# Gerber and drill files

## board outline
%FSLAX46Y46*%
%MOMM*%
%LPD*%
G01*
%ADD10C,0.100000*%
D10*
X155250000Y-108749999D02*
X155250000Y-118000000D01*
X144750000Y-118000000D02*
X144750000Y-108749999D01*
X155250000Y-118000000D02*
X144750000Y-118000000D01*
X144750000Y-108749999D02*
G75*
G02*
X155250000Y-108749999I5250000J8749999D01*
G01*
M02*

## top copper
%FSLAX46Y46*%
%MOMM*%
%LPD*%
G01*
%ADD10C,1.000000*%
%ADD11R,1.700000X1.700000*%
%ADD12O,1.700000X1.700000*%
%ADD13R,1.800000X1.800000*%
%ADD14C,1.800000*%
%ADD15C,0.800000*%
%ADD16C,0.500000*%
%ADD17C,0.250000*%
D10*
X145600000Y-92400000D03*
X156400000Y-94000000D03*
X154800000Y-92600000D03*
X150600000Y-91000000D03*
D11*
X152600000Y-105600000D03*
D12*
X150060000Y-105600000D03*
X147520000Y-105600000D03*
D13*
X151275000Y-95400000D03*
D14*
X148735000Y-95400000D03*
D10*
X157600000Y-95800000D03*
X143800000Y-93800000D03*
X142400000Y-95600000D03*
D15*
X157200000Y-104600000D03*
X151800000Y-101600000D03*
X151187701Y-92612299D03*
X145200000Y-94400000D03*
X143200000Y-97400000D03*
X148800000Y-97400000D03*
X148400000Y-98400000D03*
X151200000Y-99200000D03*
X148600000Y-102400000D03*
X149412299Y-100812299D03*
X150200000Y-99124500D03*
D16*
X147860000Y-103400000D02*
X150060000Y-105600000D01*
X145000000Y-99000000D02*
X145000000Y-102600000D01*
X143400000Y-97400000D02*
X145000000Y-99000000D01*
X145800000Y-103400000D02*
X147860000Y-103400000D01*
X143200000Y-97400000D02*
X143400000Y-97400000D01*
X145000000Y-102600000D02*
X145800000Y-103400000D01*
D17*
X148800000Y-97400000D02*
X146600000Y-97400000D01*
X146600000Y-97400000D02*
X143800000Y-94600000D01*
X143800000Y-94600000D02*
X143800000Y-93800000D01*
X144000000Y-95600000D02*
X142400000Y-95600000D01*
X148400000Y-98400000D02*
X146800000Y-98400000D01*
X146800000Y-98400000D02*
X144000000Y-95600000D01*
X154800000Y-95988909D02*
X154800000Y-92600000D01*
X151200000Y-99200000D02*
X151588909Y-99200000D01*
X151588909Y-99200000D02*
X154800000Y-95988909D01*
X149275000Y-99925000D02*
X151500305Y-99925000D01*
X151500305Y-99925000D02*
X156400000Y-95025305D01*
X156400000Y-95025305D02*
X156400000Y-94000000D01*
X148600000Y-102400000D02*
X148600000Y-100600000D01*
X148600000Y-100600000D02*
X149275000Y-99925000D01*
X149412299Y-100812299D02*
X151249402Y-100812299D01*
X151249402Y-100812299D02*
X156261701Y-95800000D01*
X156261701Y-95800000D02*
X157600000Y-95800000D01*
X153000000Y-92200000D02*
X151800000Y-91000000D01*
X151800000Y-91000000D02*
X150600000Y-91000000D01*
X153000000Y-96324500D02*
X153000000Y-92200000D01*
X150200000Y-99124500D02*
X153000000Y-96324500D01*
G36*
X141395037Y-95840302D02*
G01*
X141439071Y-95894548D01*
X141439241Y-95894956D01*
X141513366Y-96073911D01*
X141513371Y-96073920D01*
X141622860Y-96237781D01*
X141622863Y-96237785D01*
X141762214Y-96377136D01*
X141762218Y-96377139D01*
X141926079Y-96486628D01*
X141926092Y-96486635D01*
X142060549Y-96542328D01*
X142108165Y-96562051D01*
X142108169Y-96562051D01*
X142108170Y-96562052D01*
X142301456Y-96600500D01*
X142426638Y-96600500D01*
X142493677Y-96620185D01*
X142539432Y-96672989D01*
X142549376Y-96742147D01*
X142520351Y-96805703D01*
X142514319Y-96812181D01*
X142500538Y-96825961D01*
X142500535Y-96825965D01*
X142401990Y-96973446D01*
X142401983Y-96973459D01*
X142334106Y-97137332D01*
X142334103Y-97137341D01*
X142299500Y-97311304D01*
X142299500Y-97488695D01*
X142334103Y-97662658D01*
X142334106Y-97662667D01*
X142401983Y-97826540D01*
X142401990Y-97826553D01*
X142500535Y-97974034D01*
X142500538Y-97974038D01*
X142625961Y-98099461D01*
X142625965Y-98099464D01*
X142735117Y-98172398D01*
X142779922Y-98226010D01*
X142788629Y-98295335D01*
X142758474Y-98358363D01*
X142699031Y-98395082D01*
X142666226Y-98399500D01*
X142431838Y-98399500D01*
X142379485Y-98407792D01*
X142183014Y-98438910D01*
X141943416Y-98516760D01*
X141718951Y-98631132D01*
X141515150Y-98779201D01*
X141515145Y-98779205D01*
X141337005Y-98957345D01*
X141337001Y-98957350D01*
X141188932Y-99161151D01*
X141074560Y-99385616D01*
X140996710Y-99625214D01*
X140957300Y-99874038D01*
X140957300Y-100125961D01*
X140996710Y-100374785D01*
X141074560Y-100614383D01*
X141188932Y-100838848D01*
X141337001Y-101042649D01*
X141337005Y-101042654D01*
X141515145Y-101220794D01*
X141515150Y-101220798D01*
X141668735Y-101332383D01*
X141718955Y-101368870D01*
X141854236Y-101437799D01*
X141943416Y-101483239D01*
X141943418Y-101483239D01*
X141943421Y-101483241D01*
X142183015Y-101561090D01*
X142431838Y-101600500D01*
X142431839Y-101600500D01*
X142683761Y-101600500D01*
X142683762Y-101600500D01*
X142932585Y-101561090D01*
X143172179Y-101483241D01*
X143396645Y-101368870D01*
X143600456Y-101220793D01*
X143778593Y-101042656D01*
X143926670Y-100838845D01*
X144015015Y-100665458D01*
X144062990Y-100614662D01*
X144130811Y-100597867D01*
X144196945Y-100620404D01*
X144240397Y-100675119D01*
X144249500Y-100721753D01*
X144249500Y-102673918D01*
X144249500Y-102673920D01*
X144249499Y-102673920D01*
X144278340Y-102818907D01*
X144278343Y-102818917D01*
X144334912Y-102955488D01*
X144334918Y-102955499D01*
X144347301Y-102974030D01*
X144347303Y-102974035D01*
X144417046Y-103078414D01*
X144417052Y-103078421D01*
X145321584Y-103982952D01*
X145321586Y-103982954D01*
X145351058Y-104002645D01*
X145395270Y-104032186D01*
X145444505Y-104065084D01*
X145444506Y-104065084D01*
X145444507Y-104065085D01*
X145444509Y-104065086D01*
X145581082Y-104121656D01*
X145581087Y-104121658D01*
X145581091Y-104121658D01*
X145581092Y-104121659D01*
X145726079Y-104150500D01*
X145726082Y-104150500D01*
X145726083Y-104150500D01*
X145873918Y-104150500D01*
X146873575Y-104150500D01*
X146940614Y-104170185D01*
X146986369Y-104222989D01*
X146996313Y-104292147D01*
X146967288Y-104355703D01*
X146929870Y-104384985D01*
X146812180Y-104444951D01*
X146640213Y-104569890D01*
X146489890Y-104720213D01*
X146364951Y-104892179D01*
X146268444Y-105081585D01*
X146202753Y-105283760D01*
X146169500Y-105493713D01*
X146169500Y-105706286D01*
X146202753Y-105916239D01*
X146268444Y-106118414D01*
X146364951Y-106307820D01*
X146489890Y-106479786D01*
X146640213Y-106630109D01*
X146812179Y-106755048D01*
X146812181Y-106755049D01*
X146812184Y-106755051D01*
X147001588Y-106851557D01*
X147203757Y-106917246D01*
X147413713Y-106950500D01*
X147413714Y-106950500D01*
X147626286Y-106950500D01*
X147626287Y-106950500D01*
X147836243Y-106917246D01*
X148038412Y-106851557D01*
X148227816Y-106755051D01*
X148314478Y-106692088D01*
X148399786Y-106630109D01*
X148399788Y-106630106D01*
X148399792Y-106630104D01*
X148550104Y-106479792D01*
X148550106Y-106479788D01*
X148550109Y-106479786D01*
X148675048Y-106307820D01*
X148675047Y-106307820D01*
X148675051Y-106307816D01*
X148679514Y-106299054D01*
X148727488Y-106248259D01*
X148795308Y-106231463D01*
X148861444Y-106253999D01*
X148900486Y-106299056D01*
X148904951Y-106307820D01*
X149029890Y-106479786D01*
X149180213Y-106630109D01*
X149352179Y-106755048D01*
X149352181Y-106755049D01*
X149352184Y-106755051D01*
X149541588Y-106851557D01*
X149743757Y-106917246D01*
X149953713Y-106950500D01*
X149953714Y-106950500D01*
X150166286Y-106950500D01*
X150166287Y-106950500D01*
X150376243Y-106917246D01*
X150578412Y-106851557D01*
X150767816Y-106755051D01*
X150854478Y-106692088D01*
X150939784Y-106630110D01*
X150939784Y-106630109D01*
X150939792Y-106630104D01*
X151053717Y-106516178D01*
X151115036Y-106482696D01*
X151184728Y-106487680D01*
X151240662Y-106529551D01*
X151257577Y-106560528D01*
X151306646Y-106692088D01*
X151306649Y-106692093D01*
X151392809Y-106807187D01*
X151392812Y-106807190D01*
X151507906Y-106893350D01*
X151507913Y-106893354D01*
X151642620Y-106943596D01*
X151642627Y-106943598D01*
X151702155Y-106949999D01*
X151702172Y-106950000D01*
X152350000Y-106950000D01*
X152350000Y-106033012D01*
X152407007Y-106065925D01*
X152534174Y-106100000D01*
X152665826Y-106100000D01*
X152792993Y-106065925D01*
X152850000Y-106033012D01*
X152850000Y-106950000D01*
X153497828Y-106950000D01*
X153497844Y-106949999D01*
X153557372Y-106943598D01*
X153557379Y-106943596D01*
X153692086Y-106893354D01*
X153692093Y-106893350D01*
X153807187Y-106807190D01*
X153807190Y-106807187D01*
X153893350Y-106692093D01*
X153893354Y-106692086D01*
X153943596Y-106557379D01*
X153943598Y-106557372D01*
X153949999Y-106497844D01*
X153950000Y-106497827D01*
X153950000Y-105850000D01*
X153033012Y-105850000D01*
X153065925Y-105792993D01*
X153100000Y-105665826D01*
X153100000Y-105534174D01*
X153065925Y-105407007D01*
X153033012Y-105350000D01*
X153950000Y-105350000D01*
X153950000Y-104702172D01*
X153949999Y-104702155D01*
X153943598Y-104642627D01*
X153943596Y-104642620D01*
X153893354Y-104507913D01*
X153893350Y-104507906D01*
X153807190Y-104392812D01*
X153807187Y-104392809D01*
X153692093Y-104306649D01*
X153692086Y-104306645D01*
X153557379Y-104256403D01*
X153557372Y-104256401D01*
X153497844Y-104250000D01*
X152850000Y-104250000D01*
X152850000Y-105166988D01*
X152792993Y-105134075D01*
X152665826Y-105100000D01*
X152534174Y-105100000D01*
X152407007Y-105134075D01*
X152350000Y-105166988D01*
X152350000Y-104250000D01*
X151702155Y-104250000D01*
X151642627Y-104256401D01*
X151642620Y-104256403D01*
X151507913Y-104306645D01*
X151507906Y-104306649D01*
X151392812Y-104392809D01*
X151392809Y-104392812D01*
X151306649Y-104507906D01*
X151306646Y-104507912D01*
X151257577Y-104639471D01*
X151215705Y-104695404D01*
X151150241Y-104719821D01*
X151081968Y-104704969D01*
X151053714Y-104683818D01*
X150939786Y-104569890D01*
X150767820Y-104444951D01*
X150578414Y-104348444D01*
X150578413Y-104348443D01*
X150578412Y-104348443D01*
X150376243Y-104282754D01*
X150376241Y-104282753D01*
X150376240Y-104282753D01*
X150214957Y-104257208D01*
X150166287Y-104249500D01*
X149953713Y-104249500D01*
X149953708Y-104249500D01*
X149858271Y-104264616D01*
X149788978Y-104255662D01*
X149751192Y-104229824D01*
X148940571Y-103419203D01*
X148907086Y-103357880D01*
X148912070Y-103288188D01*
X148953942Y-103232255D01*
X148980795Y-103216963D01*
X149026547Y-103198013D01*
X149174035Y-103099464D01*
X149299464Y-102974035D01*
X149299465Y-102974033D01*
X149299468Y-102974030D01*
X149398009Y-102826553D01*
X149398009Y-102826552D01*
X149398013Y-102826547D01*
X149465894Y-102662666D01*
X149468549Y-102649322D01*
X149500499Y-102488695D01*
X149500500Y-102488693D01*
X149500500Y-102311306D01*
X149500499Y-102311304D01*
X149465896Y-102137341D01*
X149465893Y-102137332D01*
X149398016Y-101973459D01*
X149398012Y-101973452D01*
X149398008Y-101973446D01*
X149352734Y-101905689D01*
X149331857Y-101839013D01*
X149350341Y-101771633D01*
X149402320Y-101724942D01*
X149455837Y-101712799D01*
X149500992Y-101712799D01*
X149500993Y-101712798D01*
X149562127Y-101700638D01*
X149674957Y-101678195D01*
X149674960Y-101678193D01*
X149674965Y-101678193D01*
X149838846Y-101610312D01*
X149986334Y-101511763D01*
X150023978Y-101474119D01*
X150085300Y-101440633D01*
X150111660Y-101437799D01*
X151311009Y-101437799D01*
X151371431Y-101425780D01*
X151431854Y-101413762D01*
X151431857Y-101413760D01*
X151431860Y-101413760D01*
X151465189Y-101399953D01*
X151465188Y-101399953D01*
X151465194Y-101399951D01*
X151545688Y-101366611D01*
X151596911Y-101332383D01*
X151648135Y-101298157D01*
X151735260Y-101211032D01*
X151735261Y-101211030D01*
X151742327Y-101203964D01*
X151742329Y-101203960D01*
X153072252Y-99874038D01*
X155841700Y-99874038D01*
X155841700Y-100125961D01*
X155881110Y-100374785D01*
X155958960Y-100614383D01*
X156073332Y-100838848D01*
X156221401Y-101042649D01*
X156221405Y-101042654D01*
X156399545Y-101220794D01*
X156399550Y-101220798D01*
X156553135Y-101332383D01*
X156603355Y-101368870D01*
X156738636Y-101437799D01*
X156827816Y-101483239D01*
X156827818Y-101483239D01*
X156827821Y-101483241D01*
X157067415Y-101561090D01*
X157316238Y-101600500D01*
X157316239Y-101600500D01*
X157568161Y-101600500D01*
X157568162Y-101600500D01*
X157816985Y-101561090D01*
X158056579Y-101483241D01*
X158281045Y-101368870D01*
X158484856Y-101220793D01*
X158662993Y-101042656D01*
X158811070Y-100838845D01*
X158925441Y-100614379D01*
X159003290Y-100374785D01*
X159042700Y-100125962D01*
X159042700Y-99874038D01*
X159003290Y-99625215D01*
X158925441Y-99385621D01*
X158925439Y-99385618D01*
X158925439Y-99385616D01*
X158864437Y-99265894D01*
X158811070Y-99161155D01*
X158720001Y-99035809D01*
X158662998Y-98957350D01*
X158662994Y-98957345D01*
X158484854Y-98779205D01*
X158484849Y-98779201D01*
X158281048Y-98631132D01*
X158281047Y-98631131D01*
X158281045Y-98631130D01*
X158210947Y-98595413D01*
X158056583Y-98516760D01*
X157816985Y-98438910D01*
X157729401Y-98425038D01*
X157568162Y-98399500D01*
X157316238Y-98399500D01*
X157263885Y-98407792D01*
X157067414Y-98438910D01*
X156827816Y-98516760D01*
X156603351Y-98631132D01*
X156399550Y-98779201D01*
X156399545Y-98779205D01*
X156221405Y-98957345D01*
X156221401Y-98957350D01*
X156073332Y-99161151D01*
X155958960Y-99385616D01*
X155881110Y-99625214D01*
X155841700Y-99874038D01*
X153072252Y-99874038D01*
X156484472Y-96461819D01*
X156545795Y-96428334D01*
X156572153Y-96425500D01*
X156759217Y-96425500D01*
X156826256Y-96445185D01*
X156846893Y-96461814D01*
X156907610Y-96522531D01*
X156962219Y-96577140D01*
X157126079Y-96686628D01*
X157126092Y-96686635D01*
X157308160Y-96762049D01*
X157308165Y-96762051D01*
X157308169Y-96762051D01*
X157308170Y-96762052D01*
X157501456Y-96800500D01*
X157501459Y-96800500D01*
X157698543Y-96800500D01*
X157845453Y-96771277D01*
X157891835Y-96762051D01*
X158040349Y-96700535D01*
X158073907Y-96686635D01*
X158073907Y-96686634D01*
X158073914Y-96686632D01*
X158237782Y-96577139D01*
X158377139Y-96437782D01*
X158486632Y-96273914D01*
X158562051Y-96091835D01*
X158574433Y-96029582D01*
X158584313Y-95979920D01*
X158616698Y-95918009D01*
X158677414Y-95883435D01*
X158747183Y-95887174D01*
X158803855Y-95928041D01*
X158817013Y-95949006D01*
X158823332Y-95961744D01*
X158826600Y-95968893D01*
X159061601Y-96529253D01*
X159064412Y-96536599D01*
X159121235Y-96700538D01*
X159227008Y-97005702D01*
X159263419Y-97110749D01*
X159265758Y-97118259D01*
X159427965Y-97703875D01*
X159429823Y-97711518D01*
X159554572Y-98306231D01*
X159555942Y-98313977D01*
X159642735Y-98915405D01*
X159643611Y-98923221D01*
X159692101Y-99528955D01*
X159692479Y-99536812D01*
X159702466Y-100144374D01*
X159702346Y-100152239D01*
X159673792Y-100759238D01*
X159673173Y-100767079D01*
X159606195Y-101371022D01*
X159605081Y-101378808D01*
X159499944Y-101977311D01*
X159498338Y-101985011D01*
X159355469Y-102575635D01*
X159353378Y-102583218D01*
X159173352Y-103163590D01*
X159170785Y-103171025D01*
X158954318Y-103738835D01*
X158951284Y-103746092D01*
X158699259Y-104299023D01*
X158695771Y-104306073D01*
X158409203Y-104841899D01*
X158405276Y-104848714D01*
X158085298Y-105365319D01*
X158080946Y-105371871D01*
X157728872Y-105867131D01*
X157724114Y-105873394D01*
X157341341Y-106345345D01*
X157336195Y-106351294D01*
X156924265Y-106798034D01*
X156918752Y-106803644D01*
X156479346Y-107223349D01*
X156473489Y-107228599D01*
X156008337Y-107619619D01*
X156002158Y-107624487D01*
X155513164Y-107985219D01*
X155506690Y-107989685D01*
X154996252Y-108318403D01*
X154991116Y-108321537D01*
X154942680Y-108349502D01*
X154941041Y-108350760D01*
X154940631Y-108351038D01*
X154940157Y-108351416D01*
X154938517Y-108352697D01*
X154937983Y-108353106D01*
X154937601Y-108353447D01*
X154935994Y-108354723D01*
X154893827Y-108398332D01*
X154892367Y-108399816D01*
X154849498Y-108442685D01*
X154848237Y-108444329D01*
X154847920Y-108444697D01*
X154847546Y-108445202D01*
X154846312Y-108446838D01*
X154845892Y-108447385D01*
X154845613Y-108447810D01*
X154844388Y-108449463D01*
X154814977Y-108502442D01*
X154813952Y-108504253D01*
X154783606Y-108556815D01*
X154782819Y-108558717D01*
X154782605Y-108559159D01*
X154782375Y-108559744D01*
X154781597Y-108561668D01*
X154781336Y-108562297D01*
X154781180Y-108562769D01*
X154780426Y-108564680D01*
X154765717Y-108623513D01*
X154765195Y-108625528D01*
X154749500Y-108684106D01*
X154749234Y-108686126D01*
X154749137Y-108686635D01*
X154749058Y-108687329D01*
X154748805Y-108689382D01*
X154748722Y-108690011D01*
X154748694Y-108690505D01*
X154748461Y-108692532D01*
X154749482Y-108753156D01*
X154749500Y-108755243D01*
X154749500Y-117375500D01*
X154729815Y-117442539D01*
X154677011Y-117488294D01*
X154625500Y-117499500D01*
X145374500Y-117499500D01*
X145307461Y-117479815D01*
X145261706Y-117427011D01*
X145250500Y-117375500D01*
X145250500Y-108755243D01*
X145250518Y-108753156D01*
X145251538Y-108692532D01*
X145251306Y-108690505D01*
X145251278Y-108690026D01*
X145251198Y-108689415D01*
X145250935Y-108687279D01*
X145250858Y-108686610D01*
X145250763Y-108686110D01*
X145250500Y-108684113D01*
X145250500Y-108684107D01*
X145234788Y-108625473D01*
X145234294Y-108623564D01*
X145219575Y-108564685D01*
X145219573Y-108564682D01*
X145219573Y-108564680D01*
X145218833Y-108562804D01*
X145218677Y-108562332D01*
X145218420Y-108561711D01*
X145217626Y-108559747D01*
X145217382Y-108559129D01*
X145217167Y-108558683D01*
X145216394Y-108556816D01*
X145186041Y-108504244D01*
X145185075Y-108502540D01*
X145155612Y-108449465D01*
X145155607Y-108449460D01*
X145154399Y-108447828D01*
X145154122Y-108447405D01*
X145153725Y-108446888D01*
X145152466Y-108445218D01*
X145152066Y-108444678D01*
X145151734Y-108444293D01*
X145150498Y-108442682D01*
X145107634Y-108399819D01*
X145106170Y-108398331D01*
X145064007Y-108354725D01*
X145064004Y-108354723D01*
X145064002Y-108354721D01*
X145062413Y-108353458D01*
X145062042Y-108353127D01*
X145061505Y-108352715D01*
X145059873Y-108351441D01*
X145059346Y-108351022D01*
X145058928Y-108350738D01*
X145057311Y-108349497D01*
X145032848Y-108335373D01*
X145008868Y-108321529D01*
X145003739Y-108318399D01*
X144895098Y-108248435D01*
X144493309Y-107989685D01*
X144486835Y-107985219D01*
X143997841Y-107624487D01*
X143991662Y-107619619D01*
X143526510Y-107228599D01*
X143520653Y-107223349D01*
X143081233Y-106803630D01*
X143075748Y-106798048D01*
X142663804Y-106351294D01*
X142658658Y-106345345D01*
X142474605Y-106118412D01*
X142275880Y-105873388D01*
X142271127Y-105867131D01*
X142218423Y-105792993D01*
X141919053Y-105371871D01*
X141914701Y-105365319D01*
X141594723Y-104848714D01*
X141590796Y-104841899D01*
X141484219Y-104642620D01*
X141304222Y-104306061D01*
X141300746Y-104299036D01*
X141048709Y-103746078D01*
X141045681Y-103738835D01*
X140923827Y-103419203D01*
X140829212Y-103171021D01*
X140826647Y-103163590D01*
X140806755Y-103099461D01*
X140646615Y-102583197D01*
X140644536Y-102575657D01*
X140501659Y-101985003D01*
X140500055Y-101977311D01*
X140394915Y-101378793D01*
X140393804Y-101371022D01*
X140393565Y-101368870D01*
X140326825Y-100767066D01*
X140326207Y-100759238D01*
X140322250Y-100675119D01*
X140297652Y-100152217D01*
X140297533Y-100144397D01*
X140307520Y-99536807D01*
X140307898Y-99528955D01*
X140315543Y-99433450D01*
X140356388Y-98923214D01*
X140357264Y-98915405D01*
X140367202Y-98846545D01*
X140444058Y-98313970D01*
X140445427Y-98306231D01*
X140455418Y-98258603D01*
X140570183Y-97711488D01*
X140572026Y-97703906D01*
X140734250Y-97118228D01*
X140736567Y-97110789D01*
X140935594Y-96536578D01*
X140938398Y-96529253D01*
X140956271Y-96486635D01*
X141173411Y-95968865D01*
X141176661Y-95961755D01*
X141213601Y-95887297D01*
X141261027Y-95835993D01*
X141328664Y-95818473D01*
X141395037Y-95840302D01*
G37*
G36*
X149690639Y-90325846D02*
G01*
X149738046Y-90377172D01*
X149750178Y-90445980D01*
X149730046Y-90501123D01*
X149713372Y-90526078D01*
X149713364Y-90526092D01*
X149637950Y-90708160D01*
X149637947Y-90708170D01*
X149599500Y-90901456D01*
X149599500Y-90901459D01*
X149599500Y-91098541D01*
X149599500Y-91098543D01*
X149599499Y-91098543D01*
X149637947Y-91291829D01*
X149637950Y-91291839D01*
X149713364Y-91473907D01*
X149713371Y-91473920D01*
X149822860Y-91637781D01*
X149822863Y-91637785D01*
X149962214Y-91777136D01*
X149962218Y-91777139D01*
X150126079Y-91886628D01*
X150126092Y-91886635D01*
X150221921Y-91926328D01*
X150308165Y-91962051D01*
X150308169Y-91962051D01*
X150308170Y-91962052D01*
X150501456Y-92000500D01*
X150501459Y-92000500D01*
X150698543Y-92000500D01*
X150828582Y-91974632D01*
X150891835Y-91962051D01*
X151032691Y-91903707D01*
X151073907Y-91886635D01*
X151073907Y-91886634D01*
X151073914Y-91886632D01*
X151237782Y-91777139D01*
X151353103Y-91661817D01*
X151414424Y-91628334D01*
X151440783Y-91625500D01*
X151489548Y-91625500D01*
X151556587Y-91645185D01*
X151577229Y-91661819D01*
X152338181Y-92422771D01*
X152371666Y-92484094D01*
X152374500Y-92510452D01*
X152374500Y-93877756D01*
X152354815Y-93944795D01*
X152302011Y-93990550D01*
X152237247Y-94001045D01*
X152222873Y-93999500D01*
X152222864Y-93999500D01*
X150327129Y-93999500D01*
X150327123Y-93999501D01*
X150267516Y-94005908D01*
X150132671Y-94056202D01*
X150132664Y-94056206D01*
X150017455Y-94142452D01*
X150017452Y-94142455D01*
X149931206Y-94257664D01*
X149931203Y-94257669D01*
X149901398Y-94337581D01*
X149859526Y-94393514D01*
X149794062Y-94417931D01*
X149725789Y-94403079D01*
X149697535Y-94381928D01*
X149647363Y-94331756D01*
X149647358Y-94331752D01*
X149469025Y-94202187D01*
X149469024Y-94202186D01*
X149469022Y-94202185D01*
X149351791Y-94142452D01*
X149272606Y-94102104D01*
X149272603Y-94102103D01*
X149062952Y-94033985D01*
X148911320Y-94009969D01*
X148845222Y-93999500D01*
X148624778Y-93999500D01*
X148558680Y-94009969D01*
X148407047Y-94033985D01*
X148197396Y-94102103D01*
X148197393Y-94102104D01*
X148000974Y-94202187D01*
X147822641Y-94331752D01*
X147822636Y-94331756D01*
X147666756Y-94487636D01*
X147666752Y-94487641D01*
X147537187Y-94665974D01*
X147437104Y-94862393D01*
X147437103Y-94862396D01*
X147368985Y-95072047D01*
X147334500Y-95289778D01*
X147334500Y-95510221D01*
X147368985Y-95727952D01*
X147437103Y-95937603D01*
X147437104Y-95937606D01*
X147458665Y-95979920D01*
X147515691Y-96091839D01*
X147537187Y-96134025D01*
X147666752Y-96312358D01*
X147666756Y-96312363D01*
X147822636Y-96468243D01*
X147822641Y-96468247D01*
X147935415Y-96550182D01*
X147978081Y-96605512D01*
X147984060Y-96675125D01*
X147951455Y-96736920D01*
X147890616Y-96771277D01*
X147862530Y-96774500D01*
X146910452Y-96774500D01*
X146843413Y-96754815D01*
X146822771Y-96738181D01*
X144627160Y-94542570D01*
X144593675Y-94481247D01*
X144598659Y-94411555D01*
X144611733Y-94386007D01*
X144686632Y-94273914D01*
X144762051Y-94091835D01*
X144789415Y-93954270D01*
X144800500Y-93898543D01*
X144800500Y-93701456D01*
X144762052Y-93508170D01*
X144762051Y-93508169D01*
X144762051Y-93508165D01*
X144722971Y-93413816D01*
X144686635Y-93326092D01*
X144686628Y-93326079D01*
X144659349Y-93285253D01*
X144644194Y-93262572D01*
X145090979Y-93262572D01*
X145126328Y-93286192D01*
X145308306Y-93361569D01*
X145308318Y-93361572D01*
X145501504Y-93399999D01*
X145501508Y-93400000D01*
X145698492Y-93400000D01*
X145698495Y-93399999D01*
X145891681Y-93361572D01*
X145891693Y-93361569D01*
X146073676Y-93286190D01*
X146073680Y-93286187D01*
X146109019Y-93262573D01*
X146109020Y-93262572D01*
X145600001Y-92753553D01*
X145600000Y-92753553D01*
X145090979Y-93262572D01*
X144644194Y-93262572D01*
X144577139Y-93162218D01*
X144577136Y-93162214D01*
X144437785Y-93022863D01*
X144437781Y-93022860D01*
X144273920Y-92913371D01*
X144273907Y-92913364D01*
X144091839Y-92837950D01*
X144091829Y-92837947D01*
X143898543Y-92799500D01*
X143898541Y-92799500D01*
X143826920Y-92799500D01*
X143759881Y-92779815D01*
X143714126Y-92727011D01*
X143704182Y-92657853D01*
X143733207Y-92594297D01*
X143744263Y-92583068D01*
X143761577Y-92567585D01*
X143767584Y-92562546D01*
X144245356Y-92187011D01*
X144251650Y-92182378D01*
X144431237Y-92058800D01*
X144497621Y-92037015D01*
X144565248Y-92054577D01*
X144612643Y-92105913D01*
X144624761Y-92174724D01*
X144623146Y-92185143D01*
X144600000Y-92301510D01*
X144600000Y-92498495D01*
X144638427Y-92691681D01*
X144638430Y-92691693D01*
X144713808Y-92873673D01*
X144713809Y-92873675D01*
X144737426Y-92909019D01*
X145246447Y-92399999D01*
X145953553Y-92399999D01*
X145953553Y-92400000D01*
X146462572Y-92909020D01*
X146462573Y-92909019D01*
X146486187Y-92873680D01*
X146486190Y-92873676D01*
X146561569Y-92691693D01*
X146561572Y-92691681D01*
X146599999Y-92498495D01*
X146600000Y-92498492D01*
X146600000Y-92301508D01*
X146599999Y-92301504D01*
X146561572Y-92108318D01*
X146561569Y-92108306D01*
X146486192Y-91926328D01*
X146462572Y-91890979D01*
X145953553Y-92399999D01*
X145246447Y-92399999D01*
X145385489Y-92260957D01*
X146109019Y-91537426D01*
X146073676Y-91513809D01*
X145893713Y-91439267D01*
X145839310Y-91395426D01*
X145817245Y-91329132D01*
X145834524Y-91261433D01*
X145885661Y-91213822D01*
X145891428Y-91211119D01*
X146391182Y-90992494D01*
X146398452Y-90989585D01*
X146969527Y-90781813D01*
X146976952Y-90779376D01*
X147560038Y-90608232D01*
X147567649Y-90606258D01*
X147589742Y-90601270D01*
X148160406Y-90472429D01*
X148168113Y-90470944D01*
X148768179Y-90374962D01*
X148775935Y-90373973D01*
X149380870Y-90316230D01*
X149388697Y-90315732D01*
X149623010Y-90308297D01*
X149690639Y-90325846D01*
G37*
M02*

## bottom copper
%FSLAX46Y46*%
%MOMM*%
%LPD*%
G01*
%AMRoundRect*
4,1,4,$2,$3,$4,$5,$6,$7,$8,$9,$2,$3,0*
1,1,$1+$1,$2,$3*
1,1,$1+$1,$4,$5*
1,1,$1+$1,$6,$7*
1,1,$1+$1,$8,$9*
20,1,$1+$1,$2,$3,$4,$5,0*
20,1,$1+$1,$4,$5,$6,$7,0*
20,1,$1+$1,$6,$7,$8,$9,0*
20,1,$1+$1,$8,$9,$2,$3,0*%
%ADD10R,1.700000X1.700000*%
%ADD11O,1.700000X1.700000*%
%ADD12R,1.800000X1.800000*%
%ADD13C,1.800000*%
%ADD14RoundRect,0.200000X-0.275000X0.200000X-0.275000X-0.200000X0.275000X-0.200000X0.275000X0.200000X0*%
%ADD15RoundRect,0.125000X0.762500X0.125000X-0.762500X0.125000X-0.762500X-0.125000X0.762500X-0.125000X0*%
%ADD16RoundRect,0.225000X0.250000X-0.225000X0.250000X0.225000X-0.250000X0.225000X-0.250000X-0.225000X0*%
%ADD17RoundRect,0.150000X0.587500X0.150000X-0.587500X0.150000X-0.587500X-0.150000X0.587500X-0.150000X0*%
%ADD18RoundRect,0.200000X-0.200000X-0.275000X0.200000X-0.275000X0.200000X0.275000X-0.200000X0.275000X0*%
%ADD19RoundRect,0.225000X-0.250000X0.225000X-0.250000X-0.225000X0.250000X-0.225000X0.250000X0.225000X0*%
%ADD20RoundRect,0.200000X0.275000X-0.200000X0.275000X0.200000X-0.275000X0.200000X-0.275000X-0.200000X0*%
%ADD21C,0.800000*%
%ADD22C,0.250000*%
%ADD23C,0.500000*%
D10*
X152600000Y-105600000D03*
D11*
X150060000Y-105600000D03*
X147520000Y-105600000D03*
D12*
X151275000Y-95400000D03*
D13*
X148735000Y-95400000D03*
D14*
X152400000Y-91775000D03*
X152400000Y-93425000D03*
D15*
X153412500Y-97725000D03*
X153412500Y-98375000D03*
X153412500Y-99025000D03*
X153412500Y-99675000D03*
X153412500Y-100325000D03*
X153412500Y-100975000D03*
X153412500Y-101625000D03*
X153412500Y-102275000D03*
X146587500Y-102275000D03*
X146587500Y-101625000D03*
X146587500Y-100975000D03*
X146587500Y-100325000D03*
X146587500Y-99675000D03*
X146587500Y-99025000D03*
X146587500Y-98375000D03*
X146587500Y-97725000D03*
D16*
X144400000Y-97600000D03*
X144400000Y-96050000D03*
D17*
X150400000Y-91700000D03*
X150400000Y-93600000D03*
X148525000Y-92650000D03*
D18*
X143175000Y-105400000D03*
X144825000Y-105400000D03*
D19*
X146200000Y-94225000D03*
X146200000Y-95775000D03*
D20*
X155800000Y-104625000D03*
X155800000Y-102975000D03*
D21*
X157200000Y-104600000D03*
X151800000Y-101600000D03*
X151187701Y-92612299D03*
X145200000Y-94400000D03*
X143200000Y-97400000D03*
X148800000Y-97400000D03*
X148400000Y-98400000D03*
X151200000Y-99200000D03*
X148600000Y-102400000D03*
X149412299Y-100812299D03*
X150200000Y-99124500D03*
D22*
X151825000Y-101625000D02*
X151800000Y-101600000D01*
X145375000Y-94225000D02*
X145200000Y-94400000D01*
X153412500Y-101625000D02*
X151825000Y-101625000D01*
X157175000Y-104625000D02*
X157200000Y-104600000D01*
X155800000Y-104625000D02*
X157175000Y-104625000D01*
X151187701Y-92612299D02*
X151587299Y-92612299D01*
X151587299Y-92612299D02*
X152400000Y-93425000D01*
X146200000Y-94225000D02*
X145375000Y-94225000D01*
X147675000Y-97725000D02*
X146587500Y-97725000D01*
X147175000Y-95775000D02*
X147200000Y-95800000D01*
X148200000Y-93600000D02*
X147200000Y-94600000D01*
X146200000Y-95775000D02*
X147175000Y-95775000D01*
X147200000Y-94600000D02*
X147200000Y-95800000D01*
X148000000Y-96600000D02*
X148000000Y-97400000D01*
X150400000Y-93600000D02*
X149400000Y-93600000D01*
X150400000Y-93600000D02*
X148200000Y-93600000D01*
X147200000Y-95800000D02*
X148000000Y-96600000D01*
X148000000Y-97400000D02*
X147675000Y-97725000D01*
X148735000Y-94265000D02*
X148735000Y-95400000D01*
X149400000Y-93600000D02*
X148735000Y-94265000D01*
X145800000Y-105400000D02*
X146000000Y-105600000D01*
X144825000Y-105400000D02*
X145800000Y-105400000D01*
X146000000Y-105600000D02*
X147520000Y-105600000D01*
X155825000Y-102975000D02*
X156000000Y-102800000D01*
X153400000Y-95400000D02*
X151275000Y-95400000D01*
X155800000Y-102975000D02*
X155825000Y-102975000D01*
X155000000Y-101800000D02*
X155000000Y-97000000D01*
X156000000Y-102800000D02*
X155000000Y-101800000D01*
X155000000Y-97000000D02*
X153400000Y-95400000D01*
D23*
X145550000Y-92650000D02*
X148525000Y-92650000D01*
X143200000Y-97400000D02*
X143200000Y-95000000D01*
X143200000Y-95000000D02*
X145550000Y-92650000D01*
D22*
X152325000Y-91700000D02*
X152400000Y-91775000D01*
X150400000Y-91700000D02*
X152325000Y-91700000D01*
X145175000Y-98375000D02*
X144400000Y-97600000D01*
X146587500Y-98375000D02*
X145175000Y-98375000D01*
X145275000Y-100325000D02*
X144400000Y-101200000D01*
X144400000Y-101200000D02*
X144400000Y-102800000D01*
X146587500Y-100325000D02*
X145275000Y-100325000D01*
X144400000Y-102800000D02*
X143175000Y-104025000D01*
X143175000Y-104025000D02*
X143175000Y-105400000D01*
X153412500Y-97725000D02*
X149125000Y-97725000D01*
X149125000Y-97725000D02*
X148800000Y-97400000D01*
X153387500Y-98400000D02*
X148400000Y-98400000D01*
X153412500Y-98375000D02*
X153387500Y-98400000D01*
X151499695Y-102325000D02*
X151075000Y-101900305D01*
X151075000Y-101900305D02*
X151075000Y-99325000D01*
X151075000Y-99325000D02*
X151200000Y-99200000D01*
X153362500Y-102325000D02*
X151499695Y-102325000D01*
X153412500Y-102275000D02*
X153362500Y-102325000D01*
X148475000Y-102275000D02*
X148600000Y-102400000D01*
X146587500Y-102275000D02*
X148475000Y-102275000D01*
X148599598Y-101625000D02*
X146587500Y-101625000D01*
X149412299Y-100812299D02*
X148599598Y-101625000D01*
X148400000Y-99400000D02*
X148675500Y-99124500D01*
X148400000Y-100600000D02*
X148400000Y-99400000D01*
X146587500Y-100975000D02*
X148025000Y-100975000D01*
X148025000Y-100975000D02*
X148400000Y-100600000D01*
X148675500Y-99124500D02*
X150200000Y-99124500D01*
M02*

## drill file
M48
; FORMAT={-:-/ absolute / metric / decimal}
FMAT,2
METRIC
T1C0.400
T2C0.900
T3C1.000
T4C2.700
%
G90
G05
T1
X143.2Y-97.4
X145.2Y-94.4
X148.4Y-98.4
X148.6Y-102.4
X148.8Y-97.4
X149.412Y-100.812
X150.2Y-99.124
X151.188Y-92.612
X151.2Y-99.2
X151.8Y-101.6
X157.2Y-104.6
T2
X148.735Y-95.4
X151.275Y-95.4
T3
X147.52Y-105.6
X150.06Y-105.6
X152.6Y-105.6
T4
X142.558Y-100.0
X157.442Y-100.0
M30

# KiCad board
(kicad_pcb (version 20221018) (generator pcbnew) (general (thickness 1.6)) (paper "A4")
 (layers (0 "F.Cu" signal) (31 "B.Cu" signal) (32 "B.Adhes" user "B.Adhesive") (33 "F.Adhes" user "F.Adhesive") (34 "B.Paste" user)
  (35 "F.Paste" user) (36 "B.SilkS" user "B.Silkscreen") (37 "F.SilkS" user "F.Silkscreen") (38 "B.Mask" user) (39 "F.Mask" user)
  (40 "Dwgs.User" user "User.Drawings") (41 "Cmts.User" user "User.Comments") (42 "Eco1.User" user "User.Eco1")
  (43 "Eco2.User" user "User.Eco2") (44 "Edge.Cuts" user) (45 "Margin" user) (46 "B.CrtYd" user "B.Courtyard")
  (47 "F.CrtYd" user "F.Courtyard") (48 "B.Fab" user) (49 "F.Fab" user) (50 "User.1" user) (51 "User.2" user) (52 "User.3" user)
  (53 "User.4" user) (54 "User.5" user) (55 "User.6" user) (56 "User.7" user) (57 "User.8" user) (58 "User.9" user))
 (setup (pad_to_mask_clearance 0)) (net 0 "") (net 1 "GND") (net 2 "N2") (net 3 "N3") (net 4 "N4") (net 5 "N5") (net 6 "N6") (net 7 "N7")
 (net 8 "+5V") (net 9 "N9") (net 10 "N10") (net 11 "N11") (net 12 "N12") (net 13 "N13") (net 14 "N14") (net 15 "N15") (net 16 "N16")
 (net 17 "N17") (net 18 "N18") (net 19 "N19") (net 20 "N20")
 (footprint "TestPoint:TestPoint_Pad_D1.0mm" (layer "F.Cu") (at 145.6 92.4)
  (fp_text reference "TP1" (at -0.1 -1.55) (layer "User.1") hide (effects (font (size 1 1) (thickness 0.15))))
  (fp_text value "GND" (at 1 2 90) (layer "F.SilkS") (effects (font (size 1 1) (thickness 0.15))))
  (pad "1" smd circle (at 0 0) (size 1 1) (layers "F.Cu" "F.Mask") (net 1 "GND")))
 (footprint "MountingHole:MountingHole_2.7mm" (layer "F.Cu") (at 157.4422 100)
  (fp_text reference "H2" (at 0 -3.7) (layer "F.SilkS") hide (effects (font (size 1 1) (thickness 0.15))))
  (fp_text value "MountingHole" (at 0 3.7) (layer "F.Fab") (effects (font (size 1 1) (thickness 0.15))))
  (pad "" np_thru_hole circle (at 0 0) (size 2.7 2.7) (drill 2.7) (layers "*.Cu" "*.Mask")))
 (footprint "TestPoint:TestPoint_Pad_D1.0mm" (layer "F.Cu") (at 156.4 94)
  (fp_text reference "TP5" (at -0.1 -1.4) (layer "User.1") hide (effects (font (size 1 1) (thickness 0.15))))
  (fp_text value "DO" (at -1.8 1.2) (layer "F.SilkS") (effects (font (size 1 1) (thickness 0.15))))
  (pad "1" smd circle (at 0 0) (size 1 1) (layers "F.Cu" "F.Mask") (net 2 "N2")))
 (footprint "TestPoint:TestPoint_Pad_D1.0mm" (layer "F.Cu") (at 154.8 92.6)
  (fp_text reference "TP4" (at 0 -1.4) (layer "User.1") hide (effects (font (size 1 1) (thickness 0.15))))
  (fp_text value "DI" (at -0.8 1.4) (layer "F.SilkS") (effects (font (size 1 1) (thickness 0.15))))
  (pad "1" smd circle (at 0 0) (size 1 1) (layers "F.Cu" "F.Mask") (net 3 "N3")))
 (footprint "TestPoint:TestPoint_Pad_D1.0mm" (layer "F.Cu") (at 150.6 91)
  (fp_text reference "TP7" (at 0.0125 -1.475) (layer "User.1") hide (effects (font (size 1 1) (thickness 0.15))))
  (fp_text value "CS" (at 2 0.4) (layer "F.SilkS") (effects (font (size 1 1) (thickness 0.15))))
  (pad "1" smd circle (at 0 0) (size 1 1) (layers "F.Cu" "F.Mask") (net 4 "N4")))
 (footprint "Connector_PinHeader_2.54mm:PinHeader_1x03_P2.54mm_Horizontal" (layer "F.Cu") (at 152.6 105.6 -90)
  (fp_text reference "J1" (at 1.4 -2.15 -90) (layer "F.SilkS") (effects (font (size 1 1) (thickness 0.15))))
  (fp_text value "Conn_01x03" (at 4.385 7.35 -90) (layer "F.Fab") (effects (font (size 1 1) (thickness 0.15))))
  (pad "1" thru_hole rect (at 0 0 270) (size 1.7 1.7) (drill 1) (layers "*.Cu" "*.Mask") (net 1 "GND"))
  (pad "2" thru_hole oval (at 0 2.54 270) (size 1.7 1.7) (drill 1) (layers "*.Cu" "*.Mask") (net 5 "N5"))
  (pad "3" thru_hole oval (at 0 5.08 270) (size 1.7 1.7) (drill 1) (layers "*.Cu" "*.Mask") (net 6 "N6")))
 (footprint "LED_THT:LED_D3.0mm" (layer "F.Cu") (at 151.275 95.4 180)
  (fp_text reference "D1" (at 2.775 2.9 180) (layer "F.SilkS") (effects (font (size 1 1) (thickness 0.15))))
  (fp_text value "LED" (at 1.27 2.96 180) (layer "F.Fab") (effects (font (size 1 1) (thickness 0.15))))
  (pad "1" thru_hole rect (at 0 0 180) (size 1.8 1.8) (drill 0.9) (layers "*.Cu" "*.Mask") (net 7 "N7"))
  (pad "2" thru_hole circle (at 2.54 0 180) (size 1.8 1.8) (drill 0.9) (layers "*.Cu" "*.Mask") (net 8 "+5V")))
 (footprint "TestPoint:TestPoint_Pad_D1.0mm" (layer "F.Cu") (at 157.6 95.8)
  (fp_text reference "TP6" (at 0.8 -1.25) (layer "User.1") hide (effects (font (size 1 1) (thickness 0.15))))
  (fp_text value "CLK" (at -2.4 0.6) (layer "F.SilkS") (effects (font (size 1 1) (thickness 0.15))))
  (pad "1" smd circle (at 0 0) (size 1 1) (layers "F.Cu" "F.Mask") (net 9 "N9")))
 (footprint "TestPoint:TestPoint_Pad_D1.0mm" (layer "F.Cu") (at 143.8 93.8)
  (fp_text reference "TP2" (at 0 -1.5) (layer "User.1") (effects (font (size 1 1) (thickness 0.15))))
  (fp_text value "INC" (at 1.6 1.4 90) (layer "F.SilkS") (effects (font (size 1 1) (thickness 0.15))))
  (pad "1" smd circle (at 0 0) (size 1 1) (layers "F.Cu" "F.Mask") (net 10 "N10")))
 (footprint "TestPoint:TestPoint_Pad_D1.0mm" (layer "F.Cu") (at 142.4 95.6)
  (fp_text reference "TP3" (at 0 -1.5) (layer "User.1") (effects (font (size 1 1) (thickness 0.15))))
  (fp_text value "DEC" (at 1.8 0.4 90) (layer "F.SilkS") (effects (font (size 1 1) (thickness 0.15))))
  (pad "1" smd circle (at 0 0) (size 1 1) (layers "F.Cu" "F.Mask") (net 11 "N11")))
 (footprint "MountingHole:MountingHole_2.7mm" (layer "F.Cu") (at 142.5578 100)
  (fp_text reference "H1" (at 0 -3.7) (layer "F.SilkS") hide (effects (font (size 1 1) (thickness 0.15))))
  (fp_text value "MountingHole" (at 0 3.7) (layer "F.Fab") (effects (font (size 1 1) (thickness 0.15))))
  (pad "" np_thru_hole circle (at 0 0) (size 2.7 2.7) (drill 2.7) (layers "*.Cu" "*.Mask")))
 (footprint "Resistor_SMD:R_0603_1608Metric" (layer "B.Cu") (at 152.4 92.6 -90)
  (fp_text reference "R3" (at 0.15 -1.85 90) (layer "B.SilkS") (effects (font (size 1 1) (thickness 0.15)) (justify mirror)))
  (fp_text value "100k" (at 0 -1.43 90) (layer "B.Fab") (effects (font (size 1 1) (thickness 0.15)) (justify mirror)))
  (pad "1" smd roundrect (at -0.825 0 270) (size 0.8 0.95) (layers "B.Cu" "B.Paste" "B.Mask") (roundrect_rratio 0.25) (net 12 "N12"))
  (pad "2" smd roundrect (at 0.825 0 270) (size 0.8 0.95) (layers "B.Cu" "B.Paste" "B.Mask") (roundrect_rratio 0.25) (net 1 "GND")))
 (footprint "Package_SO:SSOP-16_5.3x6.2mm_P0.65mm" (layer "B.Cu") (at 150 100 180)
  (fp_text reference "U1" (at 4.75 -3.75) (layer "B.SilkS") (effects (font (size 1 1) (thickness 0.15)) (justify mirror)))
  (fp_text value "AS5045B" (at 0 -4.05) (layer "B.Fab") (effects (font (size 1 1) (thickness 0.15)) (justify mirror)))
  (pad "1" smd roundrect (at -3.4125 2.275 180) (size 1.775 0.5) (layers "B.Cu" "B.Paste" "B.Mask") (roundrect_rratio 0.25) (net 10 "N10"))
  (pad "2" smd roundrect (at -3.4125 1.625 180) (size 1.775 0.5) (layers "B.Cu" "B.Paste" "B.Mask") (roundrect_rratio 0.25) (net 11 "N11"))
  (pad "3" smd roundrect (at -3.4125 0.975 180) (size 1.775 0.5) (layers "B.Cu" "B.Paste" "B.Mask") (roundrect_rratio 0.25) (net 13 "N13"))
  (pad "4" smd roundrect (at -3.4125 0.325 180) (size 1.775 0.5) (layers "B.Cu" "B.Paste" "B.Mask") (roundrect_rratio 0.25) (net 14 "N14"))
  (pad "5" smd roundrect (at -3.4125 -0.325 180) (size 1.775 0.5) (layers "B.Cu" "B.Paste" "B.Mask") (roundrect_rratio 0.25) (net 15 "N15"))
  (pad "6" smd roundrect (at -3.4125 -0.975 180) (size 1.775 0.5) (layers "B.Cu" "B.Paste" "B.Mask") (roundrect_rratio 0.25) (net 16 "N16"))
  (pad "7" smd roundrect (at -3.4125 -1.625 180) (size 1.775 0.5) (layers "B.Cu" "B.Paste" "B.Mask") (roundrect_rratio 0.25) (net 1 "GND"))
  (pad "8" smd roundrect (at -3.4125 -2.275 180) (size 1.775 0.5) (layers "B.Cu" "B.Paste" "B.Mask") (roundrect_rratio 0.25) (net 3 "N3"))
  (pad "9" smd roundrect (at 3.4125 -2.275 180) (size 1.775 0.5) (layers "B.Cu" "B.Paste" "B.Mask") (roundrect_rratio 0.25) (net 2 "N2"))
  (pad "10" smd roundrect (at 3.4125 -1.625 180) (size 1.775 0.5) (layers "B.Cu" "B.Paste" "B.Mask") (roundrect_rratio 0.25) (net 9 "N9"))
  (pad "11" smd roundrect (at 3.4125 -0.975 180) (size 1.775 0.5) (layers "B.Cu" "B.Paste" "B.Mask") (roundrect_rratio 0.25) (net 4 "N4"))
  (pad "12" smd roundrect (at 3.4125 -0.325 180) (size 1.775 0.5) (layers "B.Cu" "B.Paste" "B.Mask") (roundrect_rratio 0.25) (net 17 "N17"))
  (pad "13" smd roundrect (at 3.4125 0.325 180) (size 1.775 0.5) (layers "B.Cu" "B.Paste" "B.Mask") (roundrect_rratio 0.25) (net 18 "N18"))
  (pad "14" smd roundrect (at 3.4125 0.975 180) (size 1.775 0.5) (layers "B.Cu" "B.Paste" "B.Mask") (roundrect_rratio 0.25) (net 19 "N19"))
  (pad "15" smd roundrect (at 3.4125 1.625 180) (size 1.775 0.5) (layers "B.Cu" "B.Paste" "B.Mask") (roundrect_rratio 0.25) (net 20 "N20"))
  (pad "16" smd roundrect (at 3.4125 2.275 180) (size 1.775 0.5) (layers "B.Cu" "B.Paste" "B.Mask") (roundrect_rratio 0.25) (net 8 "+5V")))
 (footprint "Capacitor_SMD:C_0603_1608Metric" (layer "B.Cu") (at 144.4 96.825 90)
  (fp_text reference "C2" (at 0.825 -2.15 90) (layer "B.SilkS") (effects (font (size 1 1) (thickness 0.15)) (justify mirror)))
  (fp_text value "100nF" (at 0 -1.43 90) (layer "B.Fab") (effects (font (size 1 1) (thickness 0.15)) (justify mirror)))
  (pad "1" smd roundrect (at -0.775 0 90) (size 0.9 0.95) (layers "B.Cu" "B.Paste" "B.Mask") (roundrect_rratio 0.25) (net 20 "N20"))
  (pad "2" smd roundrect (at 0.775 0 90) (size 0.9 0.95) (layers "B.Cu" "B.Paste" "B.Mask") (roundrect_rratio 0.25) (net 1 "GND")))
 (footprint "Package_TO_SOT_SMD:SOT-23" (layer "B.Cu") (at 149.4625 92.65 180)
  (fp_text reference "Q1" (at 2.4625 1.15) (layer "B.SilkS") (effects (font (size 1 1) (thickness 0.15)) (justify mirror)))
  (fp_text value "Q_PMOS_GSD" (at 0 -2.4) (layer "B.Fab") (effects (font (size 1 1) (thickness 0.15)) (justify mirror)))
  (pad "1" smd roundrect (at -0.9375 0.95 180) (size 1.475 0.6) (layers "B.Cu" "B.Paste" "B.Mask") (roundrect_rratio 0.25) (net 12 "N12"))
  (pad "2" smd roundrect (at -0.9375 -0.95 180) (size 1.475 0.6) (layers "B.Cu" "B.Paste" "B.Mask") (roundrect_rratio 0.25) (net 8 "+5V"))
  (pad "3" smd roundrect (at 0.9375 0 180) (size 1.475 0.6) (layers "B.Cu" "B.Paste" "B.Mask") (roundrect_rratio 0.25) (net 5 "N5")))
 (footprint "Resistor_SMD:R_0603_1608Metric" (layer "B.Cu") (at 144 105.4)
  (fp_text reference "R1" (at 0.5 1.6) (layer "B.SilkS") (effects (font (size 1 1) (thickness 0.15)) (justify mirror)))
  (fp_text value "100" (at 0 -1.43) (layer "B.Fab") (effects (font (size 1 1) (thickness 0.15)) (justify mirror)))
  (pad "1" smd roundrect (at -0.825 0) (size 0.8 0.95) (layers "B.Cu" "B.Paste" "B.Mask") (roundrect_rratio 0.25) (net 17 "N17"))
  (pad "2" smd roundrect (at 0.825 0) (size 0.8 0.95) (layers "B.Cu" "B.Paste" "B.Mask") (roundrect_rratio 0.25) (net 6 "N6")))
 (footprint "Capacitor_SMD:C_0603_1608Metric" (layer "B.Cu") (at 146.2 95 -90)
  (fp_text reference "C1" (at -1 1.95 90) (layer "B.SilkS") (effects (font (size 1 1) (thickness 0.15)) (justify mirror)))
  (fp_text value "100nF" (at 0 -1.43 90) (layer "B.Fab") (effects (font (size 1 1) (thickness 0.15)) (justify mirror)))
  (pad "1" smd roundrect (at -0.775 0 270) (size 0.9 0.95) (layers "B.Cu" "B.Paste" "B.Mask") (roundrect_rratio 0.25) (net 1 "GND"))
  (pad "2" smd roundrect (at 0.775 0 270) (size 0.9 0.95) (layers "B.Cu" "B.Paste" "B.Mask") (roundrect_rratio 0.25) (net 8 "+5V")))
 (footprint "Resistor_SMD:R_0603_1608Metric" (layer "B.Cu") (at 155.8 103.8 90)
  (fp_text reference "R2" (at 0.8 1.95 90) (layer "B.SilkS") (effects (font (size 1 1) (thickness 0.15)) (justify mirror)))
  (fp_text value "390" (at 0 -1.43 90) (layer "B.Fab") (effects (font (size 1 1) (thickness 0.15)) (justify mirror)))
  (pad "1" smd roundrect (at -0.825 0 90) (size 0.8 0.95) (layers "B.Cu" "B.Paste" "B.Mask") (roundrect_rratio 0.25) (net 1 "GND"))
  (pad "2" smd roundrect (at 0.825 0 90) (size 0.8 0.95) (layers "B.Cu" "B.Paste" "B.Mask") (roundrect_rratio 0.25) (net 7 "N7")))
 (gr_line (start 155.25 108.749999) (end 155.25 118) (stroke (width 0.1) (type default)) (layer "Edge.Cuts"))
 (gr_line (start 144.75 118) (end 144.75 108.749999) (stroke (width 0.1) (type default)) (layer "Edge.Cuts"))
 (gr_line (start 155.25 118) (end 144.75 118) (stroke (width 0.1) (type default)) (layer "Edge.Cuts"))
 (gr_arc (start 144.75 108.749999) (mid 150 89.795835) (end 155.25 108.749999) (stroke (width 0.1) (type default)) (layer "Edge.Cuts"))
 (via (at 157.2 104.6) (size 0.8) (drill 0.4) (layers "F.Cu" "B.Cu") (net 1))
 (via (at 151.8 101.6) (size 0.8) (drill 0.4) (layers "F.Cu" "B.Cu") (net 1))
 (via (at 151.187701 92.612299) (size 0.8) (drill 0.4) (layers "F.Cu" "B.Cu") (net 1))
 (via (at 145.2 94.4) (size 0.8) (drill 0.4) (layers "F.Cu" "B.Cu") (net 1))
 (segment (start 151.825 101.625) (end 151.8 101.6) (width 0.25) (layer "B.Cu") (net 1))
 (segment (start 145.375 94.225) (end 145.2 94.4) (width 0.25) (layer "B.Cu") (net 1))
 (segment (start 153.4125 101.625) (end 151.825 101.625) (width 0.25) (layer "B.Cu") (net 1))
 (segment (start 157.175 104.625) (end 157.2 104.6) (width 0.25) (layer "B.Cu") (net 1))
 (segment (start 155.8 104.625) (end 157.175 104.625) (width 0.25) (layer "B.Cu") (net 1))
 (segment (start 151.187701 92.612299) (end 151.587299 92.612299) (width 0.25) (layer "B.Cu") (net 1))
 (segment (start 151.587299 92.612299) (end 152.4 93.425) (width 0.25) (layer "B.Cu") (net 1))
 (segment (start 146.2 94.225) (end 145.375 94.225) (width 0.25) (layer "B.Cu") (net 1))
 (segment (start 147.675 97.725) (end 146.5875 97.725) (width 0.25) (layer "B.Cu") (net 8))
 (segment (start 147.175 95.775) (end 147.2 95.8) (width 0.25) (layer "B.Cu") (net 8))
 (segment (start 148.2 93.6) (end 147.2 94.6) (width 0.25) (layer "B.Cu") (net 8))
 (segment (start 146.2 95.775) (end 147.175 95.775) (width 0.25) (layer "B.Cu") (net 8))
 (segment (start 147.2 94.6) (end 147.2 95.8) (width 0.25) (layer "B.Cu") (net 8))
 (segment (start 148 96.6) (end 148 97.4) (width 0.25) (layer "B.Cu") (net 8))
 (segment (start 150.4 93.6) (end 149.4 93.6) (width 0.25) (layer "B.Cu") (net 8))
 (segment (start 150.4 93.6) (end 148.2 93.6) (width 0.25) (layer "B.Cu") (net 8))
 (segment (start 147.2 95.8) (end 148 96.6) (width 0.25) (layer "B.Cu") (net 8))
 (segment (start 148 97.4) (end 147.675 97.725) (width 0.25) (layer "B.Cu") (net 8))
 (segment (start 148.735 94.265) (end 148.735 95.4) (width 0.25) (layer "B.Cu") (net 8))
 (segment (start 149.4 93.6) (end 148.735 94.265) (width 0.25) (layer "B.Cu") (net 8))
 (segment (start 145.8 105.4) (end 146 105.6) (width 0.25) (layer "B.Cu") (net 6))
 (segment (start 144.825 105.4) (end 145.8 105.4) (width 0.25) (layer "B.Cu") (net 6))
 (segment (start 146 105.6) (end 147.52 105.6) (width 0.25) (layer "B.Cu") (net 6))
 (segment (start 155.825 102.975) (end 156 102.8) (width 0.25) (layer "B.Cu") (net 7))
 (segment (start 153.4 95.4) (end 151.275 95.4) (width 0.25) (layer "B.Cu") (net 7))
 (segment (start 155.8 102.975) (end 155.825 102.975) (width 0.25) (layer "B.Cu") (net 7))
 (segment (start 155 101.8) (end 155 97) (width 0.25) (layer "B.Cu") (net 7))
 (segment (start 156 102.8) (end 155 101.8) (width 0.25) (layer "B.Cu") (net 7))
 (segment (start 155 97) (end 153.4 95.4) (width 0.25) (layer "B.Cu") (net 7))
 (segment (start 147.86 103.4) (end 150.06 105.6) (width 0.5) (layer "F.Cu") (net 5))
 (segment (start 145 99) (end 145 102.6) (width 0.5) (layer "F.Cu") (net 5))
 (segment (start 143.4 97.4) (end 145 99) (width 0.5) (layer "F.Cu") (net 5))
 (segment (start 145.8 103.4) (end 147.86 103.4) (width 0.5) (layer "F.Cu") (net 5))
 (segment (start 143.2 97.4) (end 143.4 97.4) (width 0.5) (layer "F.Cu") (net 5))
 (segment (start 145 102.6) (end 145.8 103.4) (width 0.5) (layer "F.Cu") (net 5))
 (via (at 143.2 97.4) (size 0.8) (drill 0.4) (layers "F.Cu" "B.Cu") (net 5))
 (segment (start 145.55 92.65) (end 148.525 92.65) (width 0.5) (layer "B.Cu") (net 5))
 (segment (start 143.2 97.4) (end 143.2 95) (width 0.5) (layer "B.Cu") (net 5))
 (segment (start 143.2 95) (end 145.55 92.65) (width 0.5) (layer "B.Cu") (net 5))
 (segment (start 152.325 91.7) (end 152.4 91.775) (width 0.25) (layer "B.Cu") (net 12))
 (segment (start 150.4 91.7) (end 152.325 91.7) (width 0.25) (layer "B.Cu") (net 12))
 (segment (start 145.175 98.375) (end 144.4 97.6) (width 0.25) (layer "B.Cu") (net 20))
 (segment (start 146.5875 98.375) (end 145.175 98.375) (width 0.25) (layer "B.Cu") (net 20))
 (segment (start 145.275 100.325) (end 144.4 101.2) (width 0.25) (layer "B.Cu") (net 17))
 (segment (start 144.4 101.2) (end 144.4 102.8) (width 0.25) (layer "B.Cu") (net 17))
 (segment (start 146.5875 100.325) (end 145.275 100.325) (width 0.25) (layer "B.Cu") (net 17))
 (segment (start 144.4 102.8) (end 143.175 104.025) (width 0.25) (layer "B.Cu") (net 17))
 (segment (start 143.175 104.025) (end 143.175 105.4) (width 0.25) (layer "B.Cu") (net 17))
 (segment (start 148.8 97.4) (end 146.6 97.4) (width 0.25) (layer "F.Cu") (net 10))
 (segment (start 146.6 97.4) (end 143.8 94.6) (width 0.25) (layer "F.Cu") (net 10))
 (segment (start 143.8 94.6) (end 143.8 93.8) (width 0.25) (layer "F.Cu") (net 10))
 (via (at 148.8 97.4) (size 0.8) (drill 0.4) (layers "F.Cu" "B.Cu") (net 10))
 (segment (start 153.4125 97.725) (end 149.125 97.725) (width 0.25) (layer "B.Cu") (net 10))
 (segment (start 149.125 97.725) (end 148.8 97.4) (width 0.25) (layer "B.Cu") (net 10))
 (segment (start 144 95.6) (end 142.4 95.6) (width 0.25) (layer "F.Cu") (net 11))
 (segment (start 148.4 98.4) (end 146.8 98.4) (width 0.25) (layer "F.Cu") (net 11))
 (segment (start 146.8 98.4) (end 144 95.6) (width 0.25) (layer "F.Cu") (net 11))
 (via (at 148.4 98.4) (size 0.8) (drill 0.4) (layers "F.Cu" "B.Cu") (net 11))
 (segment (start 153.3875 98.4) (end 148.4 98.4) (width 0.25) (layer "B.Cu") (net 11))
 (segment (start 153.4125 98.375) (end 153.3875 98.4) (width 0.25) (layer "B.Cu") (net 11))
 (segment (start 154.8 95.988909) (end 154.8 92.6) (width 0.25) (layer "F.Cu") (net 3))
 (segment (start 151.2 99.2) (end 151.588909 99.2) (width 0.25) (layer "F.Cu") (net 3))
 (segment (start 151.588909 99.2) (end 154.8 95.988909) (width 0.25) (layer "F.Cu") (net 3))
 (via (at 151.2 99.2) (size 0.8) (drill 0.4) (layers "F.Cu" "B.Cu") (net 3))
 (segment (start 151.499695 102.325) (end 151.075 101.900305) (width 0.25) (layer "B.Cu") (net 3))
 (segment (start 151.075 101.900305) (end 151.075 99.325) (width 0.25) (layer "B.Cu") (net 3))
 (segment (start 151.075 99.325) (end 151.2 99.2) (width 0.25) (layer "B.Cu") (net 3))
 (segment (start 153.3625 102.325) (end 151.499695 102.325) (width 0.25) (layer "B.Cu") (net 3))
 (segment (start 153.4125 102.275) (end 153.3625 102.325) (width 0.25) (layer "B.Cu") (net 3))
 (segment (start 149.275 99.925) (end 151.500305 99.925) (width 0.25) (layer "F.Cu") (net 2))
 (segment (start 151.500305 99.925) (end 156.4 95.025305) (width 0.25) (layer "F.Cu") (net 2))
 (segment (start 156.4 95.025305) (end 156.4 94) (width 0.25) (layer "F.Cu") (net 2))
 (segment (start 148.6 102.4) (end 148.6 100.6) (width 0.25) (layer "F.Cu") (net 2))
 (segment (start 148.6 100.6) (end 149.275 99.925) (width 0.25) (layer "F.Cu") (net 2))
 (via (at 148.6 102.4) (size 0.8) (drill 0.4) (layers "F.Cu" "B.Cu") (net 2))
 (segment (start 148.475 102.275) (end 148.6 102.4) (width 0.25) (layer "B.Cu") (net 2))
 (segment (start 146.5875 102.275) (end 148.475 102.275) (width 0.25) (layer "B.Cu") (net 2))
 (segment (start 149.412299 100.812299) (end 151.249402 100.812299) (width 0.25) (layer "F.Cu") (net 9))
 (segment (start 151.249402 100.812299) (end 156.261701 95.8) (width 0.25) (layer "F.Cu") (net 9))
 (segment (start 156.261701 95.8) (end 157.6 95.8) (width 0.25) (layer "F.Cu") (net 9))
 (via (at 149.412299 100.812299) (size 0.8) (drill 0.4) (layers "F.Cu" "B.Cu") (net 9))
 (segment (start 148.599598 101.625) (end 146.5875 101.625) (width 0.25) (layer "B.Cu") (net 9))
 (segment (start 149.412299 100.812299) (end 148.599598 101.625) (width 0.25) (layer "B.Cu") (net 9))
 (segment (start 153 92.2) (end 151.8 91) (width 0.25) (layer "F.Cu") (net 4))
 (segment (start 151.8 91) (end 150.6 91) (width 0.25) (layer "F.Cu") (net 4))
 (segment (start 153 96.3245) (end 153 92.2) (width 0.25) (layer "F.Cu") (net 4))
 (segment (start 150.2 99.1245) (end 153 96.3245) (width 0.25) (layer "F.Cu") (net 4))
 (via (at 150.2 99.1245) (size 0.8) (drill 0.4) (layers "F.Cu" "B.Cu") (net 4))
 (segment (start 148.4 99.4) (end 148.6755 99.1245) (width 0.25) (layer "B.Cu") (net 4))
 (segment (start 148.4 100.6) (end 148.4 99.4) (width 0.25) (layer "B.Cu") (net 4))
 (segment (start 146.5875 100.975) (end 148.025 100.975) (width 0.25) (layer "B.Cu") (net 4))
 (segment (start 148.025 100.975) (end 148.4 100.6) (width 0.25) (layer "B.Cu") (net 4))
 (segment (start 148.6755 99.1245) (end 150.2 99.1245) (width 0.25) (layer "B.Cu") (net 4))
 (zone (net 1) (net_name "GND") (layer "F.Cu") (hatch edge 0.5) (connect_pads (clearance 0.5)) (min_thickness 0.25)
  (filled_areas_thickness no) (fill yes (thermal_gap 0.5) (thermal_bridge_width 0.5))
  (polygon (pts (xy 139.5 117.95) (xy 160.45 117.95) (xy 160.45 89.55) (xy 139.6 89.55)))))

